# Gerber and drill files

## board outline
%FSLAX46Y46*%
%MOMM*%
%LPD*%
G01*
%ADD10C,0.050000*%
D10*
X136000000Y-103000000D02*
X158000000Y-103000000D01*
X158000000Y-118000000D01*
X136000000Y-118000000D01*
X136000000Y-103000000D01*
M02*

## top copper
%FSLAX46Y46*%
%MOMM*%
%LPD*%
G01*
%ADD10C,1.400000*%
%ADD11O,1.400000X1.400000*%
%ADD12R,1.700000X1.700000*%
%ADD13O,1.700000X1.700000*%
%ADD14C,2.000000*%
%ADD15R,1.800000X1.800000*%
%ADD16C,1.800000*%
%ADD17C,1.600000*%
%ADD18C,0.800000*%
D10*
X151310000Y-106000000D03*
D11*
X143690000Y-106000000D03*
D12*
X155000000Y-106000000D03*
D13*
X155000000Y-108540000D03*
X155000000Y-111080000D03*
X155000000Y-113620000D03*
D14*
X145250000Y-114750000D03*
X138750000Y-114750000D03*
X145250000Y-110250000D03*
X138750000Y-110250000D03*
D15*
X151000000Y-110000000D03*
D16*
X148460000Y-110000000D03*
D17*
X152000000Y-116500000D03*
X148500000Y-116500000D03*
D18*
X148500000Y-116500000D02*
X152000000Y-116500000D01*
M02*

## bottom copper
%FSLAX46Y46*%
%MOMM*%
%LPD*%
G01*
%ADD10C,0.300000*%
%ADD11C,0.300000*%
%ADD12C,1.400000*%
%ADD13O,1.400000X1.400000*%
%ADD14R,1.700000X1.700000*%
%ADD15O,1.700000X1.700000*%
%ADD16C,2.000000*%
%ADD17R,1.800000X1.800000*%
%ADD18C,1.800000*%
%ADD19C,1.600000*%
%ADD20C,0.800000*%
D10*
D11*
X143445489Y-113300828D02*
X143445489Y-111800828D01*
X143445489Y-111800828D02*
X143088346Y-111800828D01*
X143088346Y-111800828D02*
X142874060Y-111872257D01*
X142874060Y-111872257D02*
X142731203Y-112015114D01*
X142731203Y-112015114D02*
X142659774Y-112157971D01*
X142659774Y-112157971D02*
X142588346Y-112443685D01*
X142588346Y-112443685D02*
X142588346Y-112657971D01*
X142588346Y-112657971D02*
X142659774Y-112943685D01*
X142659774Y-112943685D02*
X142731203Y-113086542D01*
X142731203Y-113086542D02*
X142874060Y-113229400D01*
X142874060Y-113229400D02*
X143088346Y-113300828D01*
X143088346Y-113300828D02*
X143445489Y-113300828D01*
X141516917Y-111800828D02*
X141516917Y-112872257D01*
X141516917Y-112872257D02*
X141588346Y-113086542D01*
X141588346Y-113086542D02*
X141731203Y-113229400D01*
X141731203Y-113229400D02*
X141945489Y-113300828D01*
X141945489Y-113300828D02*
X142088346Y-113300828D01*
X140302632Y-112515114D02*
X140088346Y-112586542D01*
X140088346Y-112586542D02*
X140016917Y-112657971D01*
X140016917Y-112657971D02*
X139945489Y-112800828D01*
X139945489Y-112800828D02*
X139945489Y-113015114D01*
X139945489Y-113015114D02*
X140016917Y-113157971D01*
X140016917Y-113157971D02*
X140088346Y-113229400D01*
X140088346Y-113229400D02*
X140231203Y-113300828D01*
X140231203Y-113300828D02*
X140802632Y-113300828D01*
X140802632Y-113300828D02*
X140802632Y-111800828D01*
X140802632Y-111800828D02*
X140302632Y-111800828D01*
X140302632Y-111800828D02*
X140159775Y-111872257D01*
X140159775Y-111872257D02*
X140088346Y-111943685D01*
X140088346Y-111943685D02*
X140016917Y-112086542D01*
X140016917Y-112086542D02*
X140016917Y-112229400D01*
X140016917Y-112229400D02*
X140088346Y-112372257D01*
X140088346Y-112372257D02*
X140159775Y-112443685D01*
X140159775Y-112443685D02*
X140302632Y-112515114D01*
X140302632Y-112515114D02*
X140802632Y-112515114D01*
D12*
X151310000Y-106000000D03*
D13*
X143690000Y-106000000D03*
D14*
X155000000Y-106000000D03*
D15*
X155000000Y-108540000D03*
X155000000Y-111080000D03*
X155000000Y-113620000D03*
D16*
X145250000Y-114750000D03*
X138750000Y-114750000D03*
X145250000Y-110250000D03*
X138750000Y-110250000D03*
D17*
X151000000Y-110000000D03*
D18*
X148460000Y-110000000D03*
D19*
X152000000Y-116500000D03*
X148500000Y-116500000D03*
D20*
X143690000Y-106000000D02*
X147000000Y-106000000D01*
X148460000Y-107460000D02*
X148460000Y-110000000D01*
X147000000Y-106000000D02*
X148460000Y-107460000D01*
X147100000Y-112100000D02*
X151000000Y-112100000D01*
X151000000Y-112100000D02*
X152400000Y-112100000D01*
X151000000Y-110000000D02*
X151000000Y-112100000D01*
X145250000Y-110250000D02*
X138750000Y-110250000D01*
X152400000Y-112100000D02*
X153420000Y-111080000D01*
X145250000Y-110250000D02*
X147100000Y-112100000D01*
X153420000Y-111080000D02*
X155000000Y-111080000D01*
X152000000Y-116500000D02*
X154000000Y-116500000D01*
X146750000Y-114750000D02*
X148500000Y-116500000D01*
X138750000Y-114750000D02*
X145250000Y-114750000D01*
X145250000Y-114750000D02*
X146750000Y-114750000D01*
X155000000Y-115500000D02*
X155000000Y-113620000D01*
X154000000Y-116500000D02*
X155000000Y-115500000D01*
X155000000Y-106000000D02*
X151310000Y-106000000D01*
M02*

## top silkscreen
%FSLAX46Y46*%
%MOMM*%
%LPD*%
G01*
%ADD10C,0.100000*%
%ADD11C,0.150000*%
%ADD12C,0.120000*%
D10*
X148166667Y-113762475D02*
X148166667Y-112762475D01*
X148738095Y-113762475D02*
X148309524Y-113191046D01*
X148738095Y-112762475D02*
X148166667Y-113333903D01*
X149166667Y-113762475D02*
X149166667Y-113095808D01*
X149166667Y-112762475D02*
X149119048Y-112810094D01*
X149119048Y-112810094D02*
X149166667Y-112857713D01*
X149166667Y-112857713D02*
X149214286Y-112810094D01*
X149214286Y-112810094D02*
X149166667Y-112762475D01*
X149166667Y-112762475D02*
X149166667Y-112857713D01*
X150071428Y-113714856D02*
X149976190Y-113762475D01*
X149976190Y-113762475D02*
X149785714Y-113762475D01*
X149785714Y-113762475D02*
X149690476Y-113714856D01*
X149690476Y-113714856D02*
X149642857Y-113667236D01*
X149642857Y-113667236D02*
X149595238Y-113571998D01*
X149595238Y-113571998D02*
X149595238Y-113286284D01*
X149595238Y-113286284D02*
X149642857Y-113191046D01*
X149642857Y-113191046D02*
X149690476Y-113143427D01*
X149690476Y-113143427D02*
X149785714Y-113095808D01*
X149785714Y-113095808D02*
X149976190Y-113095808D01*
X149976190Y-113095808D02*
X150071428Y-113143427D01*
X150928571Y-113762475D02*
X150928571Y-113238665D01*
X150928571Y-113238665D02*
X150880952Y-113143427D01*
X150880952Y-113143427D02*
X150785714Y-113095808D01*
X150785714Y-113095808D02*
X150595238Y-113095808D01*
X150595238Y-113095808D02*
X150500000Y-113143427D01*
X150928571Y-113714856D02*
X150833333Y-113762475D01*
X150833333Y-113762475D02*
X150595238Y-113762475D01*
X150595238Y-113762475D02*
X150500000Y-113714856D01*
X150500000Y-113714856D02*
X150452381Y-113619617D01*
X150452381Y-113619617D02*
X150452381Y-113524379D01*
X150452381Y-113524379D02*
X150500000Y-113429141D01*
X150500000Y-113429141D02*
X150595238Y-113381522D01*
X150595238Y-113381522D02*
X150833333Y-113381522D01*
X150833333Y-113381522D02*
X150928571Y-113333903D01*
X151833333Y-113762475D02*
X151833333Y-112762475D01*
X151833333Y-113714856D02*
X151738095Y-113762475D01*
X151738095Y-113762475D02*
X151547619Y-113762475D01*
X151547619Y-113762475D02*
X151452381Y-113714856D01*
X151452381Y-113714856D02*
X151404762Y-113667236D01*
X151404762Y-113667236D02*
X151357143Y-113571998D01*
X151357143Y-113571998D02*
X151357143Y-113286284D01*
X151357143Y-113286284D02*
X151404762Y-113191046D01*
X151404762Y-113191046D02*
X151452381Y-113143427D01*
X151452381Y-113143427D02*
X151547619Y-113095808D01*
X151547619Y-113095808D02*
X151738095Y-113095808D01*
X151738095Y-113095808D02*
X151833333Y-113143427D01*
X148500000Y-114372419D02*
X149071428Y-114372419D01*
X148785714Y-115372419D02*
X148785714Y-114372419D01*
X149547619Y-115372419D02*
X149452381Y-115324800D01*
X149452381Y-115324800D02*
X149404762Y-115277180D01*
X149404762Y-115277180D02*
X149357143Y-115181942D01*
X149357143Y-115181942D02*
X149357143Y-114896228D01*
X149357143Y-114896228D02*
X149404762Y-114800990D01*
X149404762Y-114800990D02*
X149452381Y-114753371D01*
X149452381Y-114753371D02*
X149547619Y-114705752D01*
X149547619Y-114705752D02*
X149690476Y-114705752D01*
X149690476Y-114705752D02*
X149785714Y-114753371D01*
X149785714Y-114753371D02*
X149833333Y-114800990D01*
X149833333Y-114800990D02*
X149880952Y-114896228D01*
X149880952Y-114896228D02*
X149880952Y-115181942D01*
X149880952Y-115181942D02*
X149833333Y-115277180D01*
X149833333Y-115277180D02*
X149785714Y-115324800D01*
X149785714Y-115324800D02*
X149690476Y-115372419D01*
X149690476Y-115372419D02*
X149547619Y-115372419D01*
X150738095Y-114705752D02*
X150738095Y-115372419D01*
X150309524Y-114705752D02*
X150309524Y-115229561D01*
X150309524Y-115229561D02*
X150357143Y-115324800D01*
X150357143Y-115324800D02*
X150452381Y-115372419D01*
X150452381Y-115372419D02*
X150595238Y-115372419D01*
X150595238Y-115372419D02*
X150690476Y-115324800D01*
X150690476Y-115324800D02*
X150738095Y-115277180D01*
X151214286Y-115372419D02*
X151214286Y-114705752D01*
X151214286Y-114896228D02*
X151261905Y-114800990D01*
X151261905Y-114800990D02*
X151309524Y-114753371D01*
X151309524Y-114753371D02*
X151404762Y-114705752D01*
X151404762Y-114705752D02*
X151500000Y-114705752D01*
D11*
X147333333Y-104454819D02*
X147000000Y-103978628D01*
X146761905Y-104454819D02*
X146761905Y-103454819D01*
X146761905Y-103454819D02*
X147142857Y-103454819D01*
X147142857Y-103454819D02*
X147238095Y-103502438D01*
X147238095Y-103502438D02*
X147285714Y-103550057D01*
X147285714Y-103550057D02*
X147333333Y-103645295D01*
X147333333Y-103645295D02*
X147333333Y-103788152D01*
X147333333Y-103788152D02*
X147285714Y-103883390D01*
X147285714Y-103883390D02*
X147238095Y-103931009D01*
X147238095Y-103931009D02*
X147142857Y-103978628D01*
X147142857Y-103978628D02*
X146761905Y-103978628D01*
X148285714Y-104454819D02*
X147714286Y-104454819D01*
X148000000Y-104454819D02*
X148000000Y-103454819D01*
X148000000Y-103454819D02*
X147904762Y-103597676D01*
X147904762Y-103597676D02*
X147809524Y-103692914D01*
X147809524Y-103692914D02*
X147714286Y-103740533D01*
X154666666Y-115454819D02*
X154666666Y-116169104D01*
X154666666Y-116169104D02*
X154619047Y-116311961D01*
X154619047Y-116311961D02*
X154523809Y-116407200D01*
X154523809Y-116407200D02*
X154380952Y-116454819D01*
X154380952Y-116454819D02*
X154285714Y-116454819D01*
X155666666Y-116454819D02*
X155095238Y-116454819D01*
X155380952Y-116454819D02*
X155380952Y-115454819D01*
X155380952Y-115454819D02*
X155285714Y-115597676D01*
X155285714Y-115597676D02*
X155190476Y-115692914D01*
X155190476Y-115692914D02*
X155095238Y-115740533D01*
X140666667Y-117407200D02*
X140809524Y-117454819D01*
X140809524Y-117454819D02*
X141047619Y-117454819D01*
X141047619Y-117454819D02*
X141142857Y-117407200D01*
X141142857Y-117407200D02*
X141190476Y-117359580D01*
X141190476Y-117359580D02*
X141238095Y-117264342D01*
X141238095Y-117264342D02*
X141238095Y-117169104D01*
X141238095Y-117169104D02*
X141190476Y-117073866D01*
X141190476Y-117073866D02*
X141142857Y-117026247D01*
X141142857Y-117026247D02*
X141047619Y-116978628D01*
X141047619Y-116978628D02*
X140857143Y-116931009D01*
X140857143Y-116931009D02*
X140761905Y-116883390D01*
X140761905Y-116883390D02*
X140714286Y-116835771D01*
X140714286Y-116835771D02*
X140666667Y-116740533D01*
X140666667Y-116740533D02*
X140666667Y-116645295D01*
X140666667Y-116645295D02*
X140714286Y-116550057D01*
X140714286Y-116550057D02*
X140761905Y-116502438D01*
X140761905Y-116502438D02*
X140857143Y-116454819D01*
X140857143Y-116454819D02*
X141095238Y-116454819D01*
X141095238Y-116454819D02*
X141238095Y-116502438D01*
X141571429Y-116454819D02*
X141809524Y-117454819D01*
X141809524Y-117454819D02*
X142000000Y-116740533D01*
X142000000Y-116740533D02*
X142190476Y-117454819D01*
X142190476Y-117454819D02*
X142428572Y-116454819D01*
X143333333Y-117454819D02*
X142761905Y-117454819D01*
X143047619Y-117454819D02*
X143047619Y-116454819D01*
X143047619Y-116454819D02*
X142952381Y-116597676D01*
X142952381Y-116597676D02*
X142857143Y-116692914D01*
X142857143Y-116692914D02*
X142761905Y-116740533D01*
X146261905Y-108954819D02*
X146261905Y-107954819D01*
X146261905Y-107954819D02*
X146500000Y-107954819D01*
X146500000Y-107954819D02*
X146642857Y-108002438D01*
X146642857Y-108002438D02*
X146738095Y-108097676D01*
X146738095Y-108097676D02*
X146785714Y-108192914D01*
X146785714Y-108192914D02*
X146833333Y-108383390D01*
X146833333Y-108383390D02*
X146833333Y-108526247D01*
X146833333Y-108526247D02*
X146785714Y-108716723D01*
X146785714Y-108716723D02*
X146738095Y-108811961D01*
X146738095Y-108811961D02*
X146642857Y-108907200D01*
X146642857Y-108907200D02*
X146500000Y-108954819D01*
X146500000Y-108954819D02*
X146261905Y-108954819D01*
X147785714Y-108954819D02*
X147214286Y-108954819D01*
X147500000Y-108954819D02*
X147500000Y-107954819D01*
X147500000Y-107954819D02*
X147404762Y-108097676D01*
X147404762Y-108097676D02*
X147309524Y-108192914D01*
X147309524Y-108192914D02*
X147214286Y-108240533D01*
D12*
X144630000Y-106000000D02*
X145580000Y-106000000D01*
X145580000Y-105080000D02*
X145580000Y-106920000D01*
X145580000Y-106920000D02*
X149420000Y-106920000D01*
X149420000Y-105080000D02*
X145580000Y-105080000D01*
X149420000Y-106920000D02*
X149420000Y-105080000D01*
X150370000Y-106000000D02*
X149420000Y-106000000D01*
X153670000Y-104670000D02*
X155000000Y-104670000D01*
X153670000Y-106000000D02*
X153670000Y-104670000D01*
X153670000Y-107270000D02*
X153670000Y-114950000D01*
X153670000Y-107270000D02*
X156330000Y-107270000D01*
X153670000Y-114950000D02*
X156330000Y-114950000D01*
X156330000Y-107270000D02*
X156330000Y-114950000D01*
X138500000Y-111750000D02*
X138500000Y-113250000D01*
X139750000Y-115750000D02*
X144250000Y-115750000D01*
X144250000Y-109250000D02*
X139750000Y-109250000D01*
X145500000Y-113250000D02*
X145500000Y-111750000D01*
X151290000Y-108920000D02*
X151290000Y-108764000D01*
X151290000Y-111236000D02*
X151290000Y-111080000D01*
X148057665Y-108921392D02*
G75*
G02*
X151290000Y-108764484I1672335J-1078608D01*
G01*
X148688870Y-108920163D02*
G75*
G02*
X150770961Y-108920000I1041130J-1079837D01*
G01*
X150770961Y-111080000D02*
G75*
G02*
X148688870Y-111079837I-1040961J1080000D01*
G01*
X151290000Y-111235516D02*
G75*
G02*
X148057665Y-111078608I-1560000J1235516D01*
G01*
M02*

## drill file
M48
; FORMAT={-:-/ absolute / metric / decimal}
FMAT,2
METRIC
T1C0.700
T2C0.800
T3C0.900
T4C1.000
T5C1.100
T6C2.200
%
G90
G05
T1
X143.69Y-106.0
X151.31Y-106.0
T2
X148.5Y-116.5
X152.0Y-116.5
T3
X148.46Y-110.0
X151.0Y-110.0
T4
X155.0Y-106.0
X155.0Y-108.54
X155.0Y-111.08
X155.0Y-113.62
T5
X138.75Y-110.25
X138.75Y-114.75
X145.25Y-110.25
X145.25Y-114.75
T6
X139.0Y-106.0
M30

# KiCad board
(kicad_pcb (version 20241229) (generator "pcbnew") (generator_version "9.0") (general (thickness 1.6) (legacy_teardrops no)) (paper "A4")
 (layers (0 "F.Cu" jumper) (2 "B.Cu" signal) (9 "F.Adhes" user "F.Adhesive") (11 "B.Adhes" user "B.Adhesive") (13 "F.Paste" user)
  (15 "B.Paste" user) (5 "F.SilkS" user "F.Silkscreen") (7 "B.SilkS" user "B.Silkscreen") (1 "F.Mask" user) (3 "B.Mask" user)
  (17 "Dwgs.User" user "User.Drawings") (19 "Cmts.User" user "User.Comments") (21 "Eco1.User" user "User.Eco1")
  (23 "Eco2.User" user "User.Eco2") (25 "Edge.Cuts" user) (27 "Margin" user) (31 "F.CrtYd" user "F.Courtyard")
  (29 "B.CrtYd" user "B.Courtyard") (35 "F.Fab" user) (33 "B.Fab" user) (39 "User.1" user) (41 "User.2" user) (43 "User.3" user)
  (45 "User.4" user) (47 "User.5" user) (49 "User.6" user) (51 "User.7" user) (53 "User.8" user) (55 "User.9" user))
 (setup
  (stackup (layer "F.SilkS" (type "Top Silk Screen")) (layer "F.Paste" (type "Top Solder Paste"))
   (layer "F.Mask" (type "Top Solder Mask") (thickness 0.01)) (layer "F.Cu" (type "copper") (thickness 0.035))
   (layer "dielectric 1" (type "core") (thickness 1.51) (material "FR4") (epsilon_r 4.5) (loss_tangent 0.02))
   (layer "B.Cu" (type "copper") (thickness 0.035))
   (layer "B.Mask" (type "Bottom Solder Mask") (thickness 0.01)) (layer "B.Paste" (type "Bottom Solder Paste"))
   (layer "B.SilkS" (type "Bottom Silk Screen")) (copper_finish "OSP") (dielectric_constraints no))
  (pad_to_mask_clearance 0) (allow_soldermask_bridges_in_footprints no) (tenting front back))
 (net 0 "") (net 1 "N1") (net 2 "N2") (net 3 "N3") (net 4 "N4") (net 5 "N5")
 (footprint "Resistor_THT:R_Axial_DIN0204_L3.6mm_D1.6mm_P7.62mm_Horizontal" (layer "F.Cu") (at 151.31 106 180)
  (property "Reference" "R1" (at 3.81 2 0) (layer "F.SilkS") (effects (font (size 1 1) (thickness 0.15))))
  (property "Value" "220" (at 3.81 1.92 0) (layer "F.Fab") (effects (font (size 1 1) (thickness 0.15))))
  (fp_line (start 6.68 0) (end 5.73 0) (stroke (width 0.12) (type solid)) (layer "F.SilkS"))
  (fp_line (start 5.73 0.92) (end 5.73 -0.92) (stroke (width 0.12) (type solid)) (layer "F.SilkS"))
  (fp_line (start 5.73 -0.92) (end 1.89 -0.92) (stroke (width 0.12) (type solid)) (layer "F.SilkS"))
  (fp_line (start 1.89 0.92) (end 5.73 0.92) (stroke (width 0.12) (type solid)) (layer "F.SilkS"))
  (fp_line (start 1.89 -0.92) (end 1.89 0.92) (stroke (width 0.12) (type solid)) (layer "F.SilkS"))
  (fp_line (start 0.94 0) (end 1.89 0) (stroke (width 0.12) (type solid)) (layer "F.SilkS"))
  (pad "1" thru_hole circle (at 0 0 180) (size 1.4 1.4) (drill 0.7) (layers "*.Cu" "*.Mask") (remove_unused_layers no) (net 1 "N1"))
  (pad "2" thru_hole oval (at 7.62 0 180) (size 1.4 1.4) (drill 0.7) (layers "*.Cu" "*.Mask") (remove_unused_layers no) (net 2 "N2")))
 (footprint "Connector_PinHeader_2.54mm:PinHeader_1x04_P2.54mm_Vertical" (layer "F.Cu") (at 155 106)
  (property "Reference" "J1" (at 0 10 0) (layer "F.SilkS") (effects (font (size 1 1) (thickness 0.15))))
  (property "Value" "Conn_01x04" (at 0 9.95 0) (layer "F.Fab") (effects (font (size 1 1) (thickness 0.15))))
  (fp_line (start -1.33 -1.33) (end 0 -1.33) (stroke (width 0.12) (type solid)) (layer "F.SilkS"))
  (fp_line (start -1.33 0) (end -1.33 -1.33) (stroke (width 0.12) (type solid)) (layer "F.SilkS"))
  (fp_line (start -1.33 1.27) (end -1.33 8.95) (stroke (width 0.12) (type solid)) (layer "F.SilkS"))
  (fp_line (start -1.33 1.27) (end 1.33 1.27) (stroke (width 0.12) (type solid)) (layer "F.SilkS"))
  (fp_line (start -1.33 8.95) (end 1.33 8.95) (stroke (width 0.12) (type solid)) (layer "F.SilkS"))
  (fp_line (start 1.33 1.27) (end 1.33 8.95) (stroke (width 0.12) (type solid)) (layer "F.SilkS"))
  (pad "1" thru_hole rect (at 0 0) (size 1.7 1.7) (drill 1) (layers "*.Cu" "*.Mask") (remove_unused_layers no) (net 1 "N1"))
  (pad "2" thru_hole oval (at 0 2.54) (size 1.7 1.7) (drill 1) (layers "*.Cu" "*.Mask") (remove_unused_layers no) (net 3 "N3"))
  (pad "3" thru_hole oval (at 0 5.08) (size 1.7 1.7) (drill 1) (layers "*.Cu" "*.Mask") (remove_unused_layers no) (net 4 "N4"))
  (pad "4" thru_hole oval (at 0 7.62) (size 1.7 1.7) (drill 1) (layers "*.Cu" "*.Mask") (remove_unused_layers no) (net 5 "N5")))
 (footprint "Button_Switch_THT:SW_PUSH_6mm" (layer "F.Cu") (at 145.25 114.75 180)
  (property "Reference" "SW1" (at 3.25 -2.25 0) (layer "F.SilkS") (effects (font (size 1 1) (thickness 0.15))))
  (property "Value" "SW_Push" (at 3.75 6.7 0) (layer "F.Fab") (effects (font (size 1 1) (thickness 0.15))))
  (fp_line (start 6.75 3) (end 6.75 1.5) (stroke (width 0.12) (type solid)) (layer "F.SilkS"))
  (fp_line (start 5.5 -1) (end 1 -1) (stroke (width 0.12) (type solid)) (layer "F.SilkS"))
  (fp_line (start 1 5.5) (end 5.5 5.5) (stroke (width 0.12) (type solid)) (layer "F.SilkS"))
  (fp_line (start -0.25 1.5) (end -0.25 3) (stroke (width 0.12) (type solid)) (layer "F.SilkS"))
  (pad "1" thru_hole circle (at 0 0 270) (size 2 2) (drill 1.1) (layers "*.Cu" "*.Mask") (remove_unused_layers no) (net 5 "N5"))
  (pad "1" thru_hole circle (at 6.5 0 270) (size 2 2) (drill 1.1) (layers "*.Cu" "*.Mask") (remove_unused_layers no) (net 5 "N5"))
  (pad "2" thru_hole circle (at 0 4.5 270) (size 2 2) (drill 1.1) (layers "*.Cu" "*.Mask") (remove_unused_layers no) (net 4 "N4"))
  (pad "2" thru_hole circle (at 6.5 4.5 270) (size 2 2) (drill 1.1) (layers "*.Cu" "*.Mask") (remove_unused_layers no) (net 4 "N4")))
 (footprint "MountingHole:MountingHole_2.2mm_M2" (layer "F.Cu") (at 139 106)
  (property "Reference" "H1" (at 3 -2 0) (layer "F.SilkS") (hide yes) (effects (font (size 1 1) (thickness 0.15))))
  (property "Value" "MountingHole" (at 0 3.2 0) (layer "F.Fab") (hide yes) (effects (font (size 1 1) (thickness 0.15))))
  (pad "" np_thru_hole circle (at 0 0) (size 2.2 2.2) (drill 2.2) (layers "*.Cu" "*.Mask")))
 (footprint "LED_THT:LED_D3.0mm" (layer "F.Cu") (at 151 110 180)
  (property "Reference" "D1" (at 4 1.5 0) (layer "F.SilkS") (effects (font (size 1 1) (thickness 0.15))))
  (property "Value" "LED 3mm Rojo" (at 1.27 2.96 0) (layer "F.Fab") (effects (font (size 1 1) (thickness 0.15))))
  (fp_line (start -0.29 1.08) (end -0.29 1.236) (stroke (width 0.12) (type solid)) (layer "F.SilkS"))
  (fp_line (start -0.29 -1.236) (end -0.29 -1.08) (stroke (width 0.12) (type solid)) (layer "F.SilkS"))
  (fp_arc (start 2.942335 1.078608) (mid 1.366487 1.987659) (end -0.29 1.235516) (stroke (width 0.12) (type solid)) (layer "F.SilkS"))
  (fp_arc (start 2.31113 1.079837) (mid 1.270117 1.5) (end 0.229039 1.08) (stroke (width 0.12) (type solid)) (layer "F.SilkS"))
  (fp_arc (start 0.229039 -1.08) (mid 1.270117 -1.5) (end 2.31113 -1.079837) (stroke (width 0.12) (type solid)) (layer "F.SilkS"))
  (fp_arc (start -0.29 -1.235516) (mid 1.366487 -1.987659) (end 2.942335 -1.078608) (stroke (width 0.12) (type solid)) (layer "F.SilkS"))
  (pad "1" thru_hole rect (at 0 0 180) (size 1.8 1.8) (drill 0.9) (layers "*.Cu" "*.Mask") (remove_unused_layers no) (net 4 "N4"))
  (pad "2" thru_hole circle (at 2.54 0 180) (size 1.8 1.8) (drill 0.9) (layers "*.Cu" "*.Mask") (remove_unused_layers no) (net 2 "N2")))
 (gr_rect (start 136 103) (end 158 118) (stroke (width 0.05) (type default)) (fill no) (layer "Edge.Cuts"))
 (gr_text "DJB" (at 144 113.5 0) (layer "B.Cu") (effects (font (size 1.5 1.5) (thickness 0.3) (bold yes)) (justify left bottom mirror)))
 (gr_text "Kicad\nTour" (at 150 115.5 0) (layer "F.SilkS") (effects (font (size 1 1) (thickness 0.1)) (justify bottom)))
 (segment (start 143.69 106) (end 147 106) (width 0.8) (layer "B.Cu") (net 2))
 (segment (start 148.46 107.46) (end 148.46 110) (width 0.8) (layer "B.Cu") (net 2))
 (segment (start 147 106) (end 148.46 107.46) (width 0.8) (layer "B.Cu") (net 2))
 (segment (start 147.1 112.1) (end 151 112.1) (width 0.8) (layer "B.Cu") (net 4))
 (segment (start 151 112.1) (end 152.4 112.1) (width 0.8) (layer "B.Cu") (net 4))
 (segment (start 151 110) (end 151 112.1) (width 0.8) (layer "B.Cu") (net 4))
 (segment (start 145.25 110.25) (end 138.75 110.25) (width 0.8) (layer "B.Cu") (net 4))
 (segment (start 152.4 112.1) (end 153.42 111.08) (width 0.8) (layer "B.Cu") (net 4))
 (segment (start 145.25 110.25) (end 147.1 112.1) (width 0.8) (layer "B.Cu") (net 4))
 (segment (start 153.42 111.08) (end 155 111.08) (width 0.8) (layer "B.Cu") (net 4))
 (segment (start 148.5 116.5) (end 152 116.5) (width 0.8) (layer "F.Cu") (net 5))
 (via (at 152 116.5) (size 1.6) (drill 0.8) (layers "F.Cu" "B.Cu") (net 5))
 (via (at 148.5 116.5) (size 1.6) (drill 0.8) (layers "F.Cu" "B.Cu") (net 5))
 (segment (start 152 116.5) (end 154 116.5) (width 0.8) (layer "B.Cu") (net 5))
 (segment (start 146.75 114.75) (end 148.5 116.5) (width 0.8) (layer "B.Cu") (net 5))
 (segment (start 138.75 114.75) (end 145.25 114.75) (width 0.8) (layer "B.Cu") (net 5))
 (segment (start 145.25 114.75) (end 146.75 114.75) (width 0.8) (layer "B.Cu") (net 5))
 (segment (start 155 115.5) (end 155 113.62) (width 0.8) (layer "B.Cu") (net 5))
 (segment (start 154 116.5) (end 155 115.5) (width 0.8) (layer "B.Cu") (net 5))
 (segment (start 155 106) (end 151.31 106) (width 0.8) (layer "B.Cu") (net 1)))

